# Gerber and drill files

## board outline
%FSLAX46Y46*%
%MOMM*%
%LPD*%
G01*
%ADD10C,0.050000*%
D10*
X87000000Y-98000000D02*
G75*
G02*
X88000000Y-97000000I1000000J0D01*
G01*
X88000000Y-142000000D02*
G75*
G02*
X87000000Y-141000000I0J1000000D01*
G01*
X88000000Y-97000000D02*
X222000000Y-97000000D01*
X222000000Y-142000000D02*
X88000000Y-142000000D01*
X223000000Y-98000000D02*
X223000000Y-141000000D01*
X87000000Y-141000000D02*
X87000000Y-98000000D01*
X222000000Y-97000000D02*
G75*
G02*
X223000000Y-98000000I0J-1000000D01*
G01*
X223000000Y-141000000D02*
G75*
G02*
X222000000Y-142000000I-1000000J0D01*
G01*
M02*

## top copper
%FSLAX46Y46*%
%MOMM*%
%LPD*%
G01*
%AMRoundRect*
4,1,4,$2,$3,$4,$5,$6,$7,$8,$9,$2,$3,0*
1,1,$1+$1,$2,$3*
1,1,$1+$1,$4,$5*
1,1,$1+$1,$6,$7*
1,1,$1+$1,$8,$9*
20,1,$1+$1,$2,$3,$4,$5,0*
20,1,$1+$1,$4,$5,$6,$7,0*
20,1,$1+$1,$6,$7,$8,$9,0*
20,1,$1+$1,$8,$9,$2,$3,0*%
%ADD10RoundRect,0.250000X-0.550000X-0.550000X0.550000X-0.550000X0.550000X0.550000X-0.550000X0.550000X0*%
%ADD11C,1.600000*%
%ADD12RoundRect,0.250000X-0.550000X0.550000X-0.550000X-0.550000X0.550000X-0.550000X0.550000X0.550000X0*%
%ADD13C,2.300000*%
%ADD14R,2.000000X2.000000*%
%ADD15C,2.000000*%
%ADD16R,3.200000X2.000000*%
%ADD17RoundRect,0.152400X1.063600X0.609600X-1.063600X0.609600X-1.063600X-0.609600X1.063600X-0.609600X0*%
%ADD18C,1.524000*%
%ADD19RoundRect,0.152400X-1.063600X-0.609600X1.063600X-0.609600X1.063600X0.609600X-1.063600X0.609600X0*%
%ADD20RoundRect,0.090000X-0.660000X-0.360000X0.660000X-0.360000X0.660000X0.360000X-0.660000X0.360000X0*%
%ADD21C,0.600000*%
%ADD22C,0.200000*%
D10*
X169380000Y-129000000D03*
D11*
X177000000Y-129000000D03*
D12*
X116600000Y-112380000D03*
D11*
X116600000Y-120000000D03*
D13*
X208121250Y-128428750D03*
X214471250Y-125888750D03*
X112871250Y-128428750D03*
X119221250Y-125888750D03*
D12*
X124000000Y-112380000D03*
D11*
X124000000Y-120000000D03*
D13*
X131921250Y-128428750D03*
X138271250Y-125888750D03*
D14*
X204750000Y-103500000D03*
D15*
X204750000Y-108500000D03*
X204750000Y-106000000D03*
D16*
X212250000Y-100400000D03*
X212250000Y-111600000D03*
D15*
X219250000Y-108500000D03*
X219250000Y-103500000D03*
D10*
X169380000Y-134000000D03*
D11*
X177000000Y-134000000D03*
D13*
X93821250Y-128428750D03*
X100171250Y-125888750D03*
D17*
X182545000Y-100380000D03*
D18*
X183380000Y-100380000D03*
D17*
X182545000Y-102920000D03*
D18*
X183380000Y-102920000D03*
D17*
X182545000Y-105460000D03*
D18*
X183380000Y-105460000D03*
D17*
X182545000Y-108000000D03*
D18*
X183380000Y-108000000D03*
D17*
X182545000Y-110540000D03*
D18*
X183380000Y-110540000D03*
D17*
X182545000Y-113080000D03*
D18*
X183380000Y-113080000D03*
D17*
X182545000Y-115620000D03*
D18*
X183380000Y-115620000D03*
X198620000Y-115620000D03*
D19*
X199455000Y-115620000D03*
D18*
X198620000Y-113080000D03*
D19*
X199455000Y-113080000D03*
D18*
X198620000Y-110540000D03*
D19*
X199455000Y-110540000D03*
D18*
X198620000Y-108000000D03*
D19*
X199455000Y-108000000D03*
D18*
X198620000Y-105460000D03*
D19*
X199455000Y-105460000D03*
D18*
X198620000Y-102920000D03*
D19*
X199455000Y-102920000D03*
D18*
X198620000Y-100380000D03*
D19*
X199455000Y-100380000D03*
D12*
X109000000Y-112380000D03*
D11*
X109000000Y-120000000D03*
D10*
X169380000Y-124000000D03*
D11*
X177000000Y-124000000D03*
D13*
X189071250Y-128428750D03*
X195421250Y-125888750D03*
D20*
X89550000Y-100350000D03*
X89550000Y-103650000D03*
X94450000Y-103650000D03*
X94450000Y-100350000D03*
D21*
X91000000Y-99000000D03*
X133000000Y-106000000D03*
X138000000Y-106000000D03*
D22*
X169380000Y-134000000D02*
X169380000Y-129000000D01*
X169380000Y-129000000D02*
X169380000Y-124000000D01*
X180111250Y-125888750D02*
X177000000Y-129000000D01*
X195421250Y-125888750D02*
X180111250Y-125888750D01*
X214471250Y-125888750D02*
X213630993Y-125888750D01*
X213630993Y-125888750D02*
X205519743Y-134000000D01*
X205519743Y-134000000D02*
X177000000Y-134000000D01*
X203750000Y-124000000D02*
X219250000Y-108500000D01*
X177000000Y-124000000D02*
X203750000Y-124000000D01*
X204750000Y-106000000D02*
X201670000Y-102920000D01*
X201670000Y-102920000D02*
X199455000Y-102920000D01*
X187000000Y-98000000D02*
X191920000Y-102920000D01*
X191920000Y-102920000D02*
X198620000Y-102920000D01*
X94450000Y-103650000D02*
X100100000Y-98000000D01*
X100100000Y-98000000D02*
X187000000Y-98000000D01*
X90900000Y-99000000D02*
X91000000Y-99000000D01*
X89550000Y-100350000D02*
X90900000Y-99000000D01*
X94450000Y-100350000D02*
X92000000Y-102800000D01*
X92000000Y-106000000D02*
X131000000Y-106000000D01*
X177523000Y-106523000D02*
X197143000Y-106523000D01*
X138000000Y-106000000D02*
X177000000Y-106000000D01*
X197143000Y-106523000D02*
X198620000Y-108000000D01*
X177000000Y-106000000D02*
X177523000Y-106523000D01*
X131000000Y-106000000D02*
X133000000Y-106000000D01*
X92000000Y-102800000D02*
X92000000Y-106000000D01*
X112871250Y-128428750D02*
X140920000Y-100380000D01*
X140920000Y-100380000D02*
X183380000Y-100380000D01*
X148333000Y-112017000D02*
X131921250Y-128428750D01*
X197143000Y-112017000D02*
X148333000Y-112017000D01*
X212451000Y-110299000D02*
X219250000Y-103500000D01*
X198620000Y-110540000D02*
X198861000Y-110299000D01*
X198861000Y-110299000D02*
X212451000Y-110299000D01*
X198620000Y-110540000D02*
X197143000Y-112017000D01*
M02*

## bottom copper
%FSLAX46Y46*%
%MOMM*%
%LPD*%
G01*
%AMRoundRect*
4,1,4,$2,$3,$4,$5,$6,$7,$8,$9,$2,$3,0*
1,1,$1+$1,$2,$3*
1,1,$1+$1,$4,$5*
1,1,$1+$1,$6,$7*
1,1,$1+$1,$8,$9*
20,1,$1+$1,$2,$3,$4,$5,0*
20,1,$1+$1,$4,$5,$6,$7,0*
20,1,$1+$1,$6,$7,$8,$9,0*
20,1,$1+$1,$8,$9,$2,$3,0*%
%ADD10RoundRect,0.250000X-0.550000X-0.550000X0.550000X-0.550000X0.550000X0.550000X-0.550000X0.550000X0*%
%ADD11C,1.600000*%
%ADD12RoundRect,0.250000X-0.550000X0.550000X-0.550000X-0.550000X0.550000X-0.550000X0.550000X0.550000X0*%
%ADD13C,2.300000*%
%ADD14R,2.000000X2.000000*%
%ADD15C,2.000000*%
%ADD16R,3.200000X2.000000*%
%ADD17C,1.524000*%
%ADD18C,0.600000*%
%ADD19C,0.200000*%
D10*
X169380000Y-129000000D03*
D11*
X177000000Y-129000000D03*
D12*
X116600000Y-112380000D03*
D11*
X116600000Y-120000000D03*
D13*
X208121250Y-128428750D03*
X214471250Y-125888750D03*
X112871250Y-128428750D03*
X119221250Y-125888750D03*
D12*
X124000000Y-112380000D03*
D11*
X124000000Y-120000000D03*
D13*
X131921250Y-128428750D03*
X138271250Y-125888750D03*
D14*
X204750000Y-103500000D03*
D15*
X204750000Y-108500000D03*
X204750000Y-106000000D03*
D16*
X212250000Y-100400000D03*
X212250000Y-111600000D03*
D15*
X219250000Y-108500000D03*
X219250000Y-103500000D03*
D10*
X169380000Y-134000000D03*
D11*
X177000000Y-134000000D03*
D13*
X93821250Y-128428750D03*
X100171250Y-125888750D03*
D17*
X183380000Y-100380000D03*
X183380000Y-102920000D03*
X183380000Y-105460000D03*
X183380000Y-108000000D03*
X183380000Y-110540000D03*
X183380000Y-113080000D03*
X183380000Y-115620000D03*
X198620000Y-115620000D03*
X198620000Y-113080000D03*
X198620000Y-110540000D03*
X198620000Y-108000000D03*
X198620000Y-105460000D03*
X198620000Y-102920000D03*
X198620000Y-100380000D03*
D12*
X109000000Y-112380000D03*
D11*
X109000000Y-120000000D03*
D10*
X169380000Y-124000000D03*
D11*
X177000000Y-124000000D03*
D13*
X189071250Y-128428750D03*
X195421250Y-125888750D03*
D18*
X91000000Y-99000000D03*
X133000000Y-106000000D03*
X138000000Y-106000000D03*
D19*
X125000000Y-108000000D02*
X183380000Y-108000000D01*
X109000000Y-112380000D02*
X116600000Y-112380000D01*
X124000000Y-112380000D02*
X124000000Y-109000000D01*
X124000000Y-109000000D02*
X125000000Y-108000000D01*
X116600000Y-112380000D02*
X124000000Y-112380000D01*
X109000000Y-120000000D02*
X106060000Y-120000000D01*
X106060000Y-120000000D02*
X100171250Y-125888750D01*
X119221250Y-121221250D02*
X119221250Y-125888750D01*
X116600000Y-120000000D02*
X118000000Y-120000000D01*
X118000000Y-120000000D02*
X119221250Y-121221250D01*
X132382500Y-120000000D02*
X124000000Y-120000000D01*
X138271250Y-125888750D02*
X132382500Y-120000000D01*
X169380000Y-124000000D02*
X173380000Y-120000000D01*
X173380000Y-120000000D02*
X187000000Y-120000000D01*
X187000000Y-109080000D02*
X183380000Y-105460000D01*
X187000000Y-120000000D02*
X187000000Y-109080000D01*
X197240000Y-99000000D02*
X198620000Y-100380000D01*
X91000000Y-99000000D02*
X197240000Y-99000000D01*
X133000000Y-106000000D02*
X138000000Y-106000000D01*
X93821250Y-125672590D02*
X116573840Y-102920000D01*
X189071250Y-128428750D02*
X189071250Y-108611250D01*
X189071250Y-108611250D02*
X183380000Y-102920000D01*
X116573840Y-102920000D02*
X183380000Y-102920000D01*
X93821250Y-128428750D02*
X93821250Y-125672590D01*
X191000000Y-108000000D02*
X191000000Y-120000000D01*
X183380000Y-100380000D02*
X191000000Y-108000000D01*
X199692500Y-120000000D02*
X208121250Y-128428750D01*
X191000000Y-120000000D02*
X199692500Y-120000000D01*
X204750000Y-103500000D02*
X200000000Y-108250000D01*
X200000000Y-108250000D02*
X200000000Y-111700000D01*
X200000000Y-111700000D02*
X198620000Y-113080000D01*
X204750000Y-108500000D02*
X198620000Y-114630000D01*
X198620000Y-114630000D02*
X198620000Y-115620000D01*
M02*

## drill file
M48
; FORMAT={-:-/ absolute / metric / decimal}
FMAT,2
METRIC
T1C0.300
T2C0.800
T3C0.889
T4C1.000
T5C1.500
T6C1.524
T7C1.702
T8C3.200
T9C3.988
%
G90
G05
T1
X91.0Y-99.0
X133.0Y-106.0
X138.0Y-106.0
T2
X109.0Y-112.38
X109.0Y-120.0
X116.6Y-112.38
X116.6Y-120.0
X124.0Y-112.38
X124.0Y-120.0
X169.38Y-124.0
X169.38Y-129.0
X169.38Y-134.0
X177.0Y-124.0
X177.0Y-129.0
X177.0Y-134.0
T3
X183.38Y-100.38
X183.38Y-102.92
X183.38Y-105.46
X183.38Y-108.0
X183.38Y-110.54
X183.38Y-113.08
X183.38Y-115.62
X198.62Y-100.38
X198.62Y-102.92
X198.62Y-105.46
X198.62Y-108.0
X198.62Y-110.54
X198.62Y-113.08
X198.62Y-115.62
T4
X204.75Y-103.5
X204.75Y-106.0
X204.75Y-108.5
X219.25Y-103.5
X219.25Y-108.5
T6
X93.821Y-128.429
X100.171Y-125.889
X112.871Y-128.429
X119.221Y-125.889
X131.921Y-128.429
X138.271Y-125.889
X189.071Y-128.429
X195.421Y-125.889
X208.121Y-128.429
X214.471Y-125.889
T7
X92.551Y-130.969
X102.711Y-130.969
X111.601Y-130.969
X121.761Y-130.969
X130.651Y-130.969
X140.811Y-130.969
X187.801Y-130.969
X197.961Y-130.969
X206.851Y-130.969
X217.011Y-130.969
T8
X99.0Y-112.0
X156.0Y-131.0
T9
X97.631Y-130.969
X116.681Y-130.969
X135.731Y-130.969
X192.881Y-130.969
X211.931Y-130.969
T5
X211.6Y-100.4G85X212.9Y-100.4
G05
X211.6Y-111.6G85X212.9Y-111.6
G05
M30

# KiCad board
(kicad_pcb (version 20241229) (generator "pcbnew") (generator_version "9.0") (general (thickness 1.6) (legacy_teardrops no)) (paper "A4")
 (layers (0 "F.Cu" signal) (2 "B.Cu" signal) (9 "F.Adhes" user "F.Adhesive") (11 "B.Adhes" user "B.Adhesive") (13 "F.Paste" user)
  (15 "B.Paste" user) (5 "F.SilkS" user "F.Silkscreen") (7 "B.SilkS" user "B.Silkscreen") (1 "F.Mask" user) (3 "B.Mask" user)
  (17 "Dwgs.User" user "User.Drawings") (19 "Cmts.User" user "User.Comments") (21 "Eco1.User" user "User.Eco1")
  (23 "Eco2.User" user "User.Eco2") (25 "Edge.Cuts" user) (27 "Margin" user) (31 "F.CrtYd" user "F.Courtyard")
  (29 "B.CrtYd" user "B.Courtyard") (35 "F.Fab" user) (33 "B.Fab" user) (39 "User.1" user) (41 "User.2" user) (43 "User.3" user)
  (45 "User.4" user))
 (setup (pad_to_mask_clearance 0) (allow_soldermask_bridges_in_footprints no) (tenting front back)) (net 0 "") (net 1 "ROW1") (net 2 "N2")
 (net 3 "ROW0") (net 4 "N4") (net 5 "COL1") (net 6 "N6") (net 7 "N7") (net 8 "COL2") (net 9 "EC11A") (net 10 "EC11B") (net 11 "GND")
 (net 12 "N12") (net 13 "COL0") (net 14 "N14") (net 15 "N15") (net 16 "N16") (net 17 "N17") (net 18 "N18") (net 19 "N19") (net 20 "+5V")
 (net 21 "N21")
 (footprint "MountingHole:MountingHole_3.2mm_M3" (layer "F.Cu") (at 99 112)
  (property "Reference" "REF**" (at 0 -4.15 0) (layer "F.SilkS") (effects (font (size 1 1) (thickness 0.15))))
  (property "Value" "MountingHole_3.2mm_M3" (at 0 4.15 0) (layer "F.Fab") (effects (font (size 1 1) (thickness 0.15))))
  (pad "" np_thru_hole circle (at 0 0) (size 3.2 3.2) (drill 3.2) (layers "*.Cu" "*.Mask")))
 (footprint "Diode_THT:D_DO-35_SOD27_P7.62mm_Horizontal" (layer "F.Cu") (at 169.38 129)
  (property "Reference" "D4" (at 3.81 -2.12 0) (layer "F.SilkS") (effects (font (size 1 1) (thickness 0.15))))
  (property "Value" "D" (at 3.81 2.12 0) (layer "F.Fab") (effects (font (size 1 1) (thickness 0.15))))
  (pad "1" thru_hole roundrect (at 0 0) (size 1.6 1.6) (drill 0.8) (layers "*.Cu" "*.Mask") (remove_unused_layers no)
   (roundrect_rratio 0.15625) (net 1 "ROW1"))
  (pad "2" thru_hole circle (at 7.62 0) (size 1.6 1.6) (drill 0.8) (layers "*.Cu" "*.Mask") (remove_unused_layers no) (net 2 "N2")))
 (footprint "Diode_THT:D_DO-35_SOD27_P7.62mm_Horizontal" (layer "F.Cu") (at 116.6 112.38 -90)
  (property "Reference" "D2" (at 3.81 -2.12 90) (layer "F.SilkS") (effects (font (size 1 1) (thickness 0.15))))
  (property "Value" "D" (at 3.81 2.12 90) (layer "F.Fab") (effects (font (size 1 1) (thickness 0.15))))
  (pad "1" thru_hole roundrect (at 0 0 270) (size 1.6 1.6) (drill 0.8) (layers "*.Cu" "*.Mask") (remove_unused_layers no)
   (roundrect_rratio 0.15625) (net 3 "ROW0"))
  (pad "2" thru_hole circle (at 7.62 0 270) (size 1.6 1.6) (drill 0.8) (layers "*.Cu" "*.Mask") (remove_unused_layers no) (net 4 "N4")))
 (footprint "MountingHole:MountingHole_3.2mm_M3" (layer "F.Cu") (at 156 131)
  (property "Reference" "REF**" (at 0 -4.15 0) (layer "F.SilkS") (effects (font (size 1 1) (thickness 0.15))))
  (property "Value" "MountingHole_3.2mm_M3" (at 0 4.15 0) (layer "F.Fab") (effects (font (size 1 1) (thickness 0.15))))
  (pad "" np_thru_hole circle (at 0 0) (size 3.2 3.2) (drill 3.2) (layers "*.Cu" "*.Mask")))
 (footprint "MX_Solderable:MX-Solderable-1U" (layer "F.Cu") (at 211.93125 130.96875)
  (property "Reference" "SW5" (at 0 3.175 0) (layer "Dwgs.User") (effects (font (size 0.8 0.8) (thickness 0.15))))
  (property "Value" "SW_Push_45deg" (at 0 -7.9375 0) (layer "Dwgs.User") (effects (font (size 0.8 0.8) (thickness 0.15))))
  (pad "" np_thru_hole circle (at -5.08 0 48.099) (size 1.7018 1.7018) (drill 1.7018) (layers "*.Cu" "*.Mask"))
  (pad "" np_thru_hole circle (at 0 0) (size 3.9878 3.9878) (drill 3.9878) (layers "*.Cu" "*.Mask"))
  (pad "" np_thru_hole circle (at 5.08 0 48.099) (size 1.7018 1.7018) (drill 1.7018) (layers "*.Cu" "*.Mask"))
  (pad "1" thru_hole circle (at -3.81 -2.54) (size 2.3 2.3) (drill 1.524) (layers "*.Cu" "B.Mask") (remove_unused_layers no) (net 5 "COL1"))
  (pad "2" thru_hole circle (at 2.54 -5.08) (size 2.3 2.3) (drill 1.524) (layers "*.Cu" "B.Mask") (remove_unused_layers no) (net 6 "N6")))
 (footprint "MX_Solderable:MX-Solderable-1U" (layer "F.Cu") (at 116.68125 130.96875)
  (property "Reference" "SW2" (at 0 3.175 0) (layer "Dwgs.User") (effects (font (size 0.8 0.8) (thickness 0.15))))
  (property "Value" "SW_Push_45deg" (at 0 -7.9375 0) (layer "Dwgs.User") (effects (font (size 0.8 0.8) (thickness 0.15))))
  (pad "" np_thru_hole circle (at -5.08 0 48.099) (size 1.7018 1.7018) (drill 1.7018) (layers "*.Cu" "*.Mask"))
  (pad "" np_thru_hole circle (at 0 0) (size 3.9878 3.9878) (drill 3.9878) (layers "*.Cu" "*.Mask"))
  (pad "" np_thru_hole circle (at 5.08 0 48.099) (size 1.7018 1.7018) (drill 1.7018) (layers "*.Cu" "*.Mask"))
  (pad "1" thru_hole circle (at -3.81 -2.54) (size 2.3 2.3) (drill 1.524) (layers "*.Cu" "B.Mask") (remove_unused_layers no) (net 5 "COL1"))
  (pad "2" thru_hole circle (at 2.54 -5.08) (size 2.3 2.3) (drill 1.524) (layers "*.Cu" "B.Mask") (remove_unused_layers no) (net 4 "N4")))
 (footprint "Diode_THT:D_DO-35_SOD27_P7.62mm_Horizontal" (layer "F.Cu") (at 124 112.38 -90)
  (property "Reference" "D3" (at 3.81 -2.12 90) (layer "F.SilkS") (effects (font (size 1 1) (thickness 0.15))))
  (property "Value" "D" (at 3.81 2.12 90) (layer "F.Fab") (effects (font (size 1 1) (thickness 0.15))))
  (pad "1" thru_hole roundrect (at 0 0 270) (size 1.6 1.6) (drill 0.8) (layers "*.Cu" "*.Mask") (remove_unused_layers no)
   (roundrect_rratio 0.15625) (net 3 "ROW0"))
  (pad "2" thru_hole circle (at 7.62 0 270) (size 1.6 1.6) (drill 0.8) (layers "*.Cu" "*.Mask") (remove_unused_layers no) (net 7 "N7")))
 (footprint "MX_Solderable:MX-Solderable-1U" (layer "F.Cu") (at 135.73125 130.96875)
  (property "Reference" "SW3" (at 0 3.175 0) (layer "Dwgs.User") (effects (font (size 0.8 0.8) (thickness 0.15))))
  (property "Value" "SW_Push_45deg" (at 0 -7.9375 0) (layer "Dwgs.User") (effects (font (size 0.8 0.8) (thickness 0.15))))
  (pad "" np_thru_hole circle (at -5.08 0 48.099) (size 1.7018 1.7018) (drill 1.7018) (layers "*.Cu" "*.Mask"))
  (pad "" np_thru_hole circle (at 0 0) (size 3.9878 3.9878) (drill 3.9878) (layers "*.Cu" "*.Mask"))
  (pad "" np_thru_hole circle (at 5.08 0 48.099) (size 1.7018 1.7018) (drill 1.7018) (layers "*.Cu" "*.Mask"))
  (pad "1" thru_hole circle (at -3.81 -2.54) (size 2.3 2.3) (drill 1.524) (layers "*.Cu" "B.Mask") (remove_unused_layers no) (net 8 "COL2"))
  (pad "2" thru_hole circle (at 2.54 -5.08) (size 2.3 2.3) (drill 1.524) (layers "*.Cu" "B.Mask") (remove_unused_layers no) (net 7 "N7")))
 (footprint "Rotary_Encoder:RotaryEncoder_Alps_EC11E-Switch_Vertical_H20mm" (layer "F.Cu") (at 204.75 103.5)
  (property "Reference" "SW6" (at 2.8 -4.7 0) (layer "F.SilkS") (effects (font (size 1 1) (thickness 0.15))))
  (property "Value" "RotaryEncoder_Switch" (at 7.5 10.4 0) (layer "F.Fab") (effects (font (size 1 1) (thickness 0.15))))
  (pad "A" thru_hole rect (at 0 0) (size 2 2) (drill 1) (layers "*.Cu" "*.Mask") (remove_unused_layers no) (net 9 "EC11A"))
  (pad "B" thru_hole circle (at 0 5) (size 2 2) (drill 1) (layers "*.Cu" "*.Mask") (remove_unused_layers no) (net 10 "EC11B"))
  (pad "C" thru_hole circle (at 0 2.5) (size 2 2) (drill 1) (layers "*.Cu" "*.Mask") (remove_unused_layers no) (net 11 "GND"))
  (pad "MP" thru_hole rect (at 7.5 -3.1) (size 3.2 2) (drill oval 2.8 1.5) (layers "*.Cu" "*.Mask") (remove_unused_layers no))
  (pad "MP" thru_hole rect (at 7.5 8.1) (size 3.2 2) (drill oval 2.8 1.5) (layers "*.Cu" "*.Mask") (remove_unused_layers no))
  (pad "S1" thru_hole circle (at 14.5 5) (size 2 2) (drill 1) (layers "*.Cu" "*.Mask") (remove_unused_layers no) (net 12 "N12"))
  (pad "S2" thru_hole circle (at 14.5 0) (size 2 2) (drill 1) (layers "*.Cu" "*.Mask") (remove_unused_layers no) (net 8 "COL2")))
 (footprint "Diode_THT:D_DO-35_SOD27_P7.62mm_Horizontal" (layer "F.Cu") (at 169.38 134)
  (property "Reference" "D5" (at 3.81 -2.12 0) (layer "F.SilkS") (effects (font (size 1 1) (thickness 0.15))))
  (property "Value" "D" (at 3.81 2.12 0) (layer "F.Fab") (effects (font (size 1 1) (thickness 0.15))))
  (pad "1" thru_hole roundrect (at 0 0) (size 1.6 1.6) (drill 0.8) (layers "*.Cu" "*.Mask") (remove_unused_layers no)
   (roundrect_rratio 0.15625) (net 1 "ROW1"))
  (pad "2" thru_hole circle (at 7.62 0) (size 1.6 1.6) (drill 0.8) (layers "*.Cu" "*.Mask") (remove_unused_layers no) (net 6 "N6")))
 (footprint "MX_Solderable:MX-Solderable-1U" (layer "F.Cu") (at 97.63125 130.96875)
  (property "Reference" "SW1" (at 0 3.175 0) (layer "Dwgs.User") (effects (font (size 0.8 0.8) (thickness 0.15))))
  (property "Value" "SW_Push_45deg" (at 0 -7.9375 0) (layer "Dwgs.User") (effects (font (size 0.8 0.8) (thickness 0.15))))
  (pad "" np_thru_hole circle (at -5.08 0 48.099) (size 1.7018 1.7018) (drill 1.7018) (layers "*.Cu" "*.Mask"))
  (pad "" np_thru_hole circle (at 0 0) (size 3.9878 3.9878) (drill 3.9878) (layers "*.Cu" "*.Mask"))
  (pad "" np_thru_hole circle (at 5.08 0 48.099) (size 1.7018 1.7018) (drill 1.7018) (layers "*.Cu" "*.Mask"))
  (pad "1" thru_hole circle (at -3.81 -2.54) (size 2.3 2.3) (drill 1.524) (layers "*.Cu" "B.Mask") (remove_unused_layers no) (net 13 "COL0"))
  (pad "2" thru_hole circle (at 2.54 -5.08) (size 2.3 2.3) (drill 1.524) (layers "*.Cu" "B.Mask") (remove_unused_layers no) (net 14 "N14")))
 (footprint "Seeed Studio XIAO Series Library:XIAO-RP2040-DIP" (layer "F.Cu") (at 191 108)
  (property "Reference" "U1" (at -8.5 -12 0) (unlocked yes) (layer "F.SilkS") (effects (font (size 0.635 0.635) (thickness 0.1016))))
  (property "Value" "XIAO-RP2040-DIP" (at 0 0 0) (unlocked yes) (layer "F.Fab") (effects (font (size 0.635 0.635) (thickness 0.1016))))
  (pad "1" smd roundrect (at -8.455 -7.62 180) (size 2.432 1.524) (layers "F.Cu" "F.Mask") (roundrect_rratio 0.1) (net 5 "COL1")
   (thermal_bridge_angle 45))
  (pad "1" thru_hole circle (at -7.62 -7.62 180) (size 1.524 1.524) (drill 0.889) (layers "*.Cu" "*.Mask") (remove_unused_layers no)
   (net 5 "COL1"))
  (pad "2" smd roundrect (at -8.455 -5.08 180) (size 2.432 1.524) (layers "F.Cu" "F.Mask") (roundrect_rratio 0.1) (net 13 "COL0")
   (thermal_bridge_angle 45))
  (pad "2" thru_hole circle (at -7.62 -5.08 180) (size 1.524 1.524) (drill 0.889) (layers "*.Cu" "*.Mask") (remove_unused_layers no)
   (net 13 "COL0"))
  (pad "3" smd roundrect (at -8.455 -2.54 180) (size 2.432 1.524) (layers "F.Cu" "F.Mask") (roundrect_rratio 0.1) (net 1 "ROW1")
   (thermal_bridge_angle 45))
  (pad "3" thru_hole circle (at -7.62 -2.54 180) (size 1.524 1.524) (drill 0.889) (layers "*.Cu" "*.Mask") (remove_unused_layers no)
   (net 1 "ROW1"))
  (pad "4" smd roundrect (at -8.455 0 180) (size 2.432 1.524) (layers "F.Cu" "F.Mask") (roundrect_rratio 0.1) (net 3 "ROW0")
   (thermal_bridge_angle 45))
  (pad "4" thru_hole circle (at -7.62 0 180) (size 1.524 1.524) (drill 0.889) (layers "*.Cu" "*.Mask") (remove_unused_layers no)
   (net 3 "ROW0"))
  (pad "5" smd roundrect (at -8.455 2.54 180) (size 2.432 1.524) (layers "F.Cu" "F.Mask") (roundrect_rratio 0.1) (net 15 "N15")
   (thermal_bridge_angle 45))
  (pad "5" thru_hole circle (at -7.62 2.54 180) (size 1.524 1.524) (drill 0.889) (layers "*.Cu" "*.Mask") (remove_unused_layers no)
   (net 15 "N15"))
  (pad "6" smd roundrect (at -8.455 5.08 180) (size 2.432 1.524) (layers "F.Cu" "F.Mask") (roundrect_rratio 0.1) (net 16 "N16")
   (thermal_bridge_angle 45))
  (pad "6" thru_hole circle (at -7.62 5.08 180) (size 1.524 1.524) (drill 0.889) (layers "*.Cu" "*.Mask") (remove_unused_layers no)
   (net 16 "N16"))
  (pad "7" smd roundrect (at -8.455 7.62 180) (size 2.432 1.524) (layers "F.Cu" "F.Mask") (roundrect_rratio 0.1) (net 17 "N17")
   (thermal_bridge_angle 45))
  (pad "7" thru_hole circle (at -7.62 7.62 180) (size 1.524 1.524) (drill 0.889) (layers "*.Cu" "*.Mask") (remove_unused_layers no)
   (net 17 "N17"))
  (pad "8" thru_hole circle (at 7.62 7.62) (size 1.524 1.524) (drill 0.889) (layers "*.Cu" "*.Mask") (remove_unused_layers no)
   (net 10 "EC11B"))
  (pad "8" smd roundrect (at 8.455 7.62) (size 2.432 1.524) (layers "F.Cu" "F.Mask") (roundrect_rratio 0.1) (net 10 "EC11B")
   (thermal_bridge_angle 45))
  (pad "9" thru_hole circle (at 7.62 5.08) (size 1.524 1.524) (drill 0.889) (layers "*.Cu" "*.Mask") (remove_unused_layers no)
   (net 9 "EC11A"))
  (pad "9" smd roundrect (at 8.455 5.08) (size 2.432 1.524) (layers "F.Cu" "F.Mask") (roundrect_rratio 0.1) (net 9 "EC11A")
   (thermal_bridge_angle 45))
  (pad "10" thru_hole circle (at 7.62 2.54) (size 1.524 1.524) (drill 0.889) (layers "*.Cu" "*.Mask") (remove_unused_layers no)
   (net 8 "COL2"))
  (pad "10" smd roundrect (at 8.455 2.54) (size 2.432 1.524) (layers "F.Cu" "F.Mask") (roundrect_rratio 0.1) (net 8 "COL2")
   (thermal_bridge_angle 45))
  (pad "11" thru_hole circle (at 7.62 0) (size 1.524 1.524) (drill 0.889) (layers "*.Cu" "*.Mask") (remove_unused_layers no) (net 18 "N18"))
  (pad "11" smd roundrect (at 8.455 0) (size 2.432 1.524) (layers "F.Cu" "F.Mask") (roundrect_rratio 0.1) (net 18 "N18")
   (thermal_bridge_angle 45))
  (pad "12" thru_hole circle (at 7.62 -2.54) (size 1.524 1.524) (drill 0.889) (layers "*.Cu" "*.Mask") (remove_unused_layers no)
   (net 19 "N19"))
  (pad "12" smd roundrect (at 8.455 -2.54) (size 2.432 1.524) (layers "F.Cu" "F.Mask") (roundrect_rratio 0.1) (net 19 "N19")
   (thermal_bridge_angle 45))
  (pad "13" thru_hole circle (at 7.62 -5.08) (size 1.524 1.524) (drill 0.889) (layers "*.Cu" "*.Mask") (remove_unused_layers no)
   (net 11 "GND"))
  (pad "13" smd roundrect (at 8.455 -5.08) (size 2.432 1.524) (layers "F.Cu" "F.Mask") (roundrect_rratio 0.1) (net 11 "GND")
   (thermal_bridge_angle 45))
  (pad "14" thru_hole circle (at 7.62 -7.62) (size 1.524 1.524) (drill 0.889) (layers "*.Cu" "*.Mask") (remove_unused_layers no)
   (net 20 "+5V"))
  (pad "14" smd roundrect (at 8.455 -7.62) (size 2.432 1.524) (layers "F.Cu" "F.Mask") (roundrect_rratio 0.1) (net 20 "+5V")
   (thermal_bridge_angle 45)))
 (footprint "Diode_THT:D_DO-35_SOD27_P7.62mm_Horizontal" (layer "F.Cu") (at 109 112.38 -90)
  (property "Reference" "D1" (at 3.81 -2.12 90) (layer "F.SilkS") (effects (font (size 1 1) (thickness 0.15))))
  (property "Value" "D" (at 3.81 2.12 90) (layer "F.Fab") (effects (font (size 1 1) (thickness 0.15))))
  (pad "1" thru_hole roundrect (at 0 0 270) (size 1.6 1.6) (drill 0.8) (layers "*.Cu" "*.Mask") (remove_unused_layers no)
   (roundrect_rratio 0.15625) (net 3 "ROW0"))
  (pad "2" thru_hole circle (at 7.62 0 270) (size 1.6 1.6) (drill 0.8) (layers "*.Cu" "*.Mask") (remove_unused_layers no) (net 14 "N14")))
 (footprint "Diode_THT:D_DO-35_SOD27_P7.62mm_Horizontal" (layer "F.Cu") (at 169.38 124)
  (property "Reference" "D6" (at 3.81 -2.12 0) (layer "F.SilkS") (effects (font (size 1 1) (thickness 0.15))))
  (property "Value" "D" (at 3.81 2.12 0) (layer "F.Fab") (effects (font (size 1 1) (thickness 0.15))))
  (pad "1" thru_hole roundrect (at 0 0) (size 1.6 1.6) (drill 0.8) (layers "*.Cu" "*.Mask") (remove_unused_layers no)
   (roundrect_rratio 0.15625) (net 1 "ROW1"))
  (pad "2" thru_hole circle (at 7.62 0) (size 1.6 1.6) (drill 0.8) (layers "*.Cu" "*.Mask") (remove_unused_layers no) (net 12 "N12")))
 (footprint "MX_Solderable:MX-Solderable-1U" (layer "F.Cu") (at 192.88125 130.96875)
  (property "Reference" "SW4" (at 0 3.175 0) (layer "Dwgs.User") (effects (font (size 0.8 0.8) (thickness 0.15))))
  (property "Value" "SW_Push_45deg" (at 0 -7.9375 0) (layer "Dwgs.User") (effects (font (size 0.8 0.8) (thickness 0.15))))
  (pad "" np_thru_hole circle (at -5.08 0 48.099) (size 1.7018 1.7018) (drill 1.7018) (layers "*.Cu" "*.Mask"))
  (pad "" np_thru_hole circle (at 0 0) (size 3.9878 3.9878) (drill 3.9878) (layers "*.Cu" "*.Mask"))
  (pad "" np_thru_hole circle (at 5.08 0 48.099) (size 1.7018 1.7018) (drill 1.7018) (layers "*.Cu" "*.Mask"))
  (pad "1" thru_hole circle (at -3.81 -2.54) (size 2.3 2.3) (drill 1.524) (layers "*.Cu" "B.Mask") (remove_unused_layers no) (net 13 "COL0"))
  (pad "2" thru_hole circle (at 2.54 -5.08) (size 2.3 2.3) (drill 1.524) (layers "*.Cu" "B.Mask") (remove_unused_layers no) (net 2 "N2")))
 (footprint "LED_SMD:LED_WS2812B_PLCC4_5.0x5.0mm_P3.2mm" (layer "F.Cu") (at 92 102)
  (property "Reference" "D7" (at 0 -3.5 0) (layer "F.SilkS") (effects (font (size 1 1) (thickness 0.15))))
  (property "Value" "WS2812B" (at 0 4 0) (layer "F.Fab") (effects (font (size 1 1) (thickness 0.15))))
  (pad "1" smd roundrect (at -2.45 -1.65) (size 1.5 0.9) (layers "F.Cu" "F.Mask" "F.Paste") (roundrect_rratio 0.1) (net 20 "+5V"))
  (pad "2" smd roundrect (at -2.45 1.65) (size 1.5 0.9) (layers "F.Cu" "F.Mask" "F.Paste") (roundrect_rratio 0.1) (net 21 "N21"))
  (pad "3" smd roundrect (at 2.45 1.65) (size 1.5 0.9) (layers "F.Cu" "F.Mask" "F.Paste") (roundrect_rratio 0.1) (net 11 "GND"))
  (pad "4" smd roundrect (at 2.45 -1.65) (size 1.5 0.9) (layers "F.Cu" "F.Mask" "F.Paste") (roundrect_rratio 0.1) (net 18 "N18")))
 (gr_arc (start 87 98) (mid 87.292893 97.292893) (end 88 97) (stroke (width 0.05) (type default)) (layer "Edge.Cuts"))
 (gr_arc (start 88 142) (mid 87.292893 141.707107) (end 87 141) (stroke (width 0.05) (type default)) (layer "Edge.Cuts"))
 (gr_line (start 88 97) (end 222 97) (stroke (width 0.05) (type default)) (layer "Edge.Cuts"))
 (gr_line (start 222 142) (end 88 142) (stroke (width 0.05) (type default)) (layer "Edge.Cuts"))
 (gr_line (start 223 98) (end 223 141) (stroke (width 0.05) (type default)) (layer "Edge.Cuts"))
 (gr_line (start 87 141) (end 87 98) (stroke (width 0.05) (type default)) (layer "Edge.Cuts"))
 (gr_arc (start 222 97) (mid 222.707107 97.292893) (end 223 98) (stroke (width 0.05) (type default)) (layer "Edge.Cuts"))
 (gr_arc (start 223 141) (mid 222.707107 141.707107) (end 222 142) (stroke (width 0.05) (type default)) (layer "Edge.Cuts"))
 (segment (start 125 108) (end 183.38 108) (width 0.2) (layer "B.Cu") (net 3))
 (segment (start 109 112.38) (end 116.6 112.38) (width 0.2) (layer "B.Cu") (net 3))
 (segment (start 124 112.38) (end 124 109) (width 0.2) (layer "B.Cu") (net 3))
 (segment (start 124 109) (end 125 108) (width 0.2) (layer "B.Cu") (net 3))
 (segment (start 116.6 112.38) (end 124 112.38) (width 0.2) (layer "B.Cu") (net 3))
 (segment (start 109 120) (end 106.06 120) (width 0.2) (layer "B.Cu") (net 14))
 (segment (start 106.06 120) (end 100.17125 125.88875) (width 0.2) (layer "B.Cu") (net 14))
 (segment (start 119.22125 121.22125) (end 119.22125 125.88875) (width 0.2) (layer "B.Cu") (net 4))
 (segment (start 116.6 120) (end 118 120) (width 0.2) (layer "B.Cu") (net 4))
 (segment (start 118 120) (end 119.22125 121.22125) (width 0.2) (layer "B.Cu") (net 4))
 (segment (start 132.3825 120) (end 124 120) (width 0.2) (layer "B.Cu") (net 7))
 (segment (start 138.27125 125.88875) (end 132.3825 120) (width 0.2) (layer "B.Cu") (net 7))
 (segment (start 169.38 134) (end 169.38 129) (width 0.2) (layer "F.Cu") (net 1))
 (segment (start 169.38 129) (end 169.38 124) (width 0.2) (layer "F.Cu") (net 1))
 (segment (start 169.38 124) (end 173.38 120) (width 0.2) (layer "B.Cu") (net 1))
 (segment (start 173.38 120) (end 187 120) (width 0.2) (layer "B.Cu") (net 1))
 (segment (start 187 109.08) (end 183.38 105.46) (width 0.2) (layer "B.Cu") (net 1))
 (segment (start 187 120) (end 187 109.08) (width 0.2) (layer "B.Cu") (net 1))
 (segment (start 180.11125 125.88875) (end 177 129) (width 0.2) (layer "F.Cu") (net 2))
 (segment (start 195.42125 125.88875) (end 180.11125 125.88875) (width 0.2) (layer "F.Cu") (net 2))
 (segment (start 214.47125 125.88875) (end 213.630993 125.88875) (width 0.2) (layer "F.Cu") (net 6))
 (segment (start 213.630993 125.88875) (end 205.519743 134) (width 0.2) (layer "F.Cu") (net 6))
 (segment (start 205.519743 134) (end 177 134) (width 0.2) (layer "F.Cu") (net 6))
 (segment (start 203.75 124) (end 219.25 108.5) (width 0.2) (layer "F.Cu") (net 12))
 (segment (start 177 124) (end 203.75 124) (width 0.2) (layer "F.Cu") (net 12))
 (segment (start 204.75 106) (end 201.67 102.92) (width 0.2) (layer "F.Cu") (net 11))
 (segment (start 201.67 102.92) (end 199.455 102.92) (width 0.2) (layer "F.Cu") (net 11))
 (segment (start 187 98) (end 191.92 102.92) (width 0.2) (layer "F.Cu") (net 11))
 (segment (start 191.92 102.92) (end 198.62 102.92) (width 0.2) (layer "F.Cu") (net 11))
 (segment (start 94.45 103.65) (end 100.1 98) (width 0.2) (layer "F.Cu") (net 11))
 (segment (start 100.1 98) (end 187 98) (width 0.2) (layer "F.Cu") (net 11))
 (segment (start 90.9 99) (end 91 99) (width 0.2) (layer "F.Cu") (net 20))
 (segment (start 89.55 100.35) (end 90.9 99) (width 0.2) (layer "F.Cu") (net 20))
 (via (at 91 99) (size 0.6) (drill 0.3) (layers "F.Cu" "B.Cu") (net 20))
 (segment (start 197.24 99) (end 198.62 100.38) (width 0.2) (layer "B.Cu") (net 20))
 (segment (start 91 99) (end 197.24 99) (width 0.2) (layer "B.Cu") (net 20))
 (segment (start 94.45 100.35) (end 92 102.8) (width 0.2) (layer "F.Cu") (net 18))
 (segment (start 92 106) (end 131 106) (width 0.2) (layer "F.Cu") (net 18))
 (segment (start 177.523 106.523) (end 197.143 106.523) (width 0.2) (layer "F.Cu") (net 18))
 (segment (start 138 106) (end 177 106) (width 0.2) (layer "F.Cu") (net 18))
 (segment (start 197.143 106.523) (end 198.62 108) (width 0.2) (layer "F.Cu") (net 18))
 (segment (start 177 106) (end 177.523 106.523) (width 0.2) (layer "F.Cu") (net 18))
 (segment (start 131 106) (end 133 106) (width 0.2) (layer "F.Cu") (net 18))
 (segment (start 92 102.8) (end 92 106) (width 0.2) (layer "F.Cu") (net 18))
 (via (at 133 106) (size 0.6) (drill 0.3) (layers "F.Cu" "B.Cu") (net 18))
 (via (at 138 106) (size 0.6) (drill 0.3) (layers "F.Cu" "B.Cu") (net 18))
 (segment (start 133 106) (end 138 106) (width 0.2) (layer "B.Cu") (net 18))
 (segment (start 93.82125 125.67259) (end 116.57384 102.92) (width 0.2) (layer "B.Cu") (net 13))
 (segment (start 189.07125 128.42875) (end 189.07125 108.61125) (width 0.2) (layer "B.Cu") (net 13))
 (segment (start 189.07125 108.61125) (end 183.38 102.92) (width 0.2) (layer "B.Cu") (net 13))
 (segment (start 116.57384 102.92) (end 183.38 102.92) (width 0.2) (layer "B.Cu") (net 13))
 (segment (start 93.82125 128.42875) (end 93.82125 125.67259) (width 0.2) (layer "B.Cu") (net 13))
 (segment (start 112.87125 128.42875) (end 140.92 100.38) (width 0.2) (layer "F.Cu") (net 5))
 (segment (start 140.92 100.38) (end 183.38 100.38) (width 0.2) (layer "F.Cu") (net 5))
 (segment (start 191 108) (end 191 120) (width 0.2) (layer "B.Cu") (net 5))
 (segment (start 183.38 100.38) (end 191 108) (width 0.2) (layer "B.Cu") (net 5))
 (segment (start 199.6925 120) (end 208.12125 128.42875) (width 0.2) (layer "B.Cu") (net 5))
 (segment (start 191 120) (end 199.6925 120) (width 0.2) (layer "B.Cu") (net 5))
 (segment (start 148.333 112.017) (end 131.92125 128.42875) (width 0.2) (layer "F.Cu") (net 8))
 (segment (start 197.143 112.017) (end 148.333 112.017) (width 0.2) (layer "F.Cu") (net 8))
 (segment (start 212.451 110.299) (end 219.25 103.5) (width 0.2) (layer "F.Cu") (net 8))
 (segment (start 198.62 110.54) (end 198.861 110.299) (width 0.2) (layer "F.Cu") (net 8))
 (segment (start 198.861 110.299) (end 212.451 110.299) (width 0.2) (layer "F.Cu") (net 8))
 (segment (start 198.62 110.54) (end 197.143 112.017) (width 0.2) (layer "F.Cu") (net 8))
 (segment (start 204.75 103.5) (end 200 108.25) (width 0.2) (layer "B.Cu") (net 9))
 (segment (start 200 108.25) (end 200 111.7) (width 0.2) (layer "B.Cu") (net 9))
 (segment (start 200 111.7) (end 198.62 113.08) (width 0.2) (layer "B.Cu") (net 9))
 (segment (start 204.75 108.5) (end 198.62 114.63) (width 0.2) (layer "B.Cu") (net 10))
 (segment (start 198.62 114.63) (end 198.62 115.62) (width 0.2) (layer "B.Cu") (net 10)))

